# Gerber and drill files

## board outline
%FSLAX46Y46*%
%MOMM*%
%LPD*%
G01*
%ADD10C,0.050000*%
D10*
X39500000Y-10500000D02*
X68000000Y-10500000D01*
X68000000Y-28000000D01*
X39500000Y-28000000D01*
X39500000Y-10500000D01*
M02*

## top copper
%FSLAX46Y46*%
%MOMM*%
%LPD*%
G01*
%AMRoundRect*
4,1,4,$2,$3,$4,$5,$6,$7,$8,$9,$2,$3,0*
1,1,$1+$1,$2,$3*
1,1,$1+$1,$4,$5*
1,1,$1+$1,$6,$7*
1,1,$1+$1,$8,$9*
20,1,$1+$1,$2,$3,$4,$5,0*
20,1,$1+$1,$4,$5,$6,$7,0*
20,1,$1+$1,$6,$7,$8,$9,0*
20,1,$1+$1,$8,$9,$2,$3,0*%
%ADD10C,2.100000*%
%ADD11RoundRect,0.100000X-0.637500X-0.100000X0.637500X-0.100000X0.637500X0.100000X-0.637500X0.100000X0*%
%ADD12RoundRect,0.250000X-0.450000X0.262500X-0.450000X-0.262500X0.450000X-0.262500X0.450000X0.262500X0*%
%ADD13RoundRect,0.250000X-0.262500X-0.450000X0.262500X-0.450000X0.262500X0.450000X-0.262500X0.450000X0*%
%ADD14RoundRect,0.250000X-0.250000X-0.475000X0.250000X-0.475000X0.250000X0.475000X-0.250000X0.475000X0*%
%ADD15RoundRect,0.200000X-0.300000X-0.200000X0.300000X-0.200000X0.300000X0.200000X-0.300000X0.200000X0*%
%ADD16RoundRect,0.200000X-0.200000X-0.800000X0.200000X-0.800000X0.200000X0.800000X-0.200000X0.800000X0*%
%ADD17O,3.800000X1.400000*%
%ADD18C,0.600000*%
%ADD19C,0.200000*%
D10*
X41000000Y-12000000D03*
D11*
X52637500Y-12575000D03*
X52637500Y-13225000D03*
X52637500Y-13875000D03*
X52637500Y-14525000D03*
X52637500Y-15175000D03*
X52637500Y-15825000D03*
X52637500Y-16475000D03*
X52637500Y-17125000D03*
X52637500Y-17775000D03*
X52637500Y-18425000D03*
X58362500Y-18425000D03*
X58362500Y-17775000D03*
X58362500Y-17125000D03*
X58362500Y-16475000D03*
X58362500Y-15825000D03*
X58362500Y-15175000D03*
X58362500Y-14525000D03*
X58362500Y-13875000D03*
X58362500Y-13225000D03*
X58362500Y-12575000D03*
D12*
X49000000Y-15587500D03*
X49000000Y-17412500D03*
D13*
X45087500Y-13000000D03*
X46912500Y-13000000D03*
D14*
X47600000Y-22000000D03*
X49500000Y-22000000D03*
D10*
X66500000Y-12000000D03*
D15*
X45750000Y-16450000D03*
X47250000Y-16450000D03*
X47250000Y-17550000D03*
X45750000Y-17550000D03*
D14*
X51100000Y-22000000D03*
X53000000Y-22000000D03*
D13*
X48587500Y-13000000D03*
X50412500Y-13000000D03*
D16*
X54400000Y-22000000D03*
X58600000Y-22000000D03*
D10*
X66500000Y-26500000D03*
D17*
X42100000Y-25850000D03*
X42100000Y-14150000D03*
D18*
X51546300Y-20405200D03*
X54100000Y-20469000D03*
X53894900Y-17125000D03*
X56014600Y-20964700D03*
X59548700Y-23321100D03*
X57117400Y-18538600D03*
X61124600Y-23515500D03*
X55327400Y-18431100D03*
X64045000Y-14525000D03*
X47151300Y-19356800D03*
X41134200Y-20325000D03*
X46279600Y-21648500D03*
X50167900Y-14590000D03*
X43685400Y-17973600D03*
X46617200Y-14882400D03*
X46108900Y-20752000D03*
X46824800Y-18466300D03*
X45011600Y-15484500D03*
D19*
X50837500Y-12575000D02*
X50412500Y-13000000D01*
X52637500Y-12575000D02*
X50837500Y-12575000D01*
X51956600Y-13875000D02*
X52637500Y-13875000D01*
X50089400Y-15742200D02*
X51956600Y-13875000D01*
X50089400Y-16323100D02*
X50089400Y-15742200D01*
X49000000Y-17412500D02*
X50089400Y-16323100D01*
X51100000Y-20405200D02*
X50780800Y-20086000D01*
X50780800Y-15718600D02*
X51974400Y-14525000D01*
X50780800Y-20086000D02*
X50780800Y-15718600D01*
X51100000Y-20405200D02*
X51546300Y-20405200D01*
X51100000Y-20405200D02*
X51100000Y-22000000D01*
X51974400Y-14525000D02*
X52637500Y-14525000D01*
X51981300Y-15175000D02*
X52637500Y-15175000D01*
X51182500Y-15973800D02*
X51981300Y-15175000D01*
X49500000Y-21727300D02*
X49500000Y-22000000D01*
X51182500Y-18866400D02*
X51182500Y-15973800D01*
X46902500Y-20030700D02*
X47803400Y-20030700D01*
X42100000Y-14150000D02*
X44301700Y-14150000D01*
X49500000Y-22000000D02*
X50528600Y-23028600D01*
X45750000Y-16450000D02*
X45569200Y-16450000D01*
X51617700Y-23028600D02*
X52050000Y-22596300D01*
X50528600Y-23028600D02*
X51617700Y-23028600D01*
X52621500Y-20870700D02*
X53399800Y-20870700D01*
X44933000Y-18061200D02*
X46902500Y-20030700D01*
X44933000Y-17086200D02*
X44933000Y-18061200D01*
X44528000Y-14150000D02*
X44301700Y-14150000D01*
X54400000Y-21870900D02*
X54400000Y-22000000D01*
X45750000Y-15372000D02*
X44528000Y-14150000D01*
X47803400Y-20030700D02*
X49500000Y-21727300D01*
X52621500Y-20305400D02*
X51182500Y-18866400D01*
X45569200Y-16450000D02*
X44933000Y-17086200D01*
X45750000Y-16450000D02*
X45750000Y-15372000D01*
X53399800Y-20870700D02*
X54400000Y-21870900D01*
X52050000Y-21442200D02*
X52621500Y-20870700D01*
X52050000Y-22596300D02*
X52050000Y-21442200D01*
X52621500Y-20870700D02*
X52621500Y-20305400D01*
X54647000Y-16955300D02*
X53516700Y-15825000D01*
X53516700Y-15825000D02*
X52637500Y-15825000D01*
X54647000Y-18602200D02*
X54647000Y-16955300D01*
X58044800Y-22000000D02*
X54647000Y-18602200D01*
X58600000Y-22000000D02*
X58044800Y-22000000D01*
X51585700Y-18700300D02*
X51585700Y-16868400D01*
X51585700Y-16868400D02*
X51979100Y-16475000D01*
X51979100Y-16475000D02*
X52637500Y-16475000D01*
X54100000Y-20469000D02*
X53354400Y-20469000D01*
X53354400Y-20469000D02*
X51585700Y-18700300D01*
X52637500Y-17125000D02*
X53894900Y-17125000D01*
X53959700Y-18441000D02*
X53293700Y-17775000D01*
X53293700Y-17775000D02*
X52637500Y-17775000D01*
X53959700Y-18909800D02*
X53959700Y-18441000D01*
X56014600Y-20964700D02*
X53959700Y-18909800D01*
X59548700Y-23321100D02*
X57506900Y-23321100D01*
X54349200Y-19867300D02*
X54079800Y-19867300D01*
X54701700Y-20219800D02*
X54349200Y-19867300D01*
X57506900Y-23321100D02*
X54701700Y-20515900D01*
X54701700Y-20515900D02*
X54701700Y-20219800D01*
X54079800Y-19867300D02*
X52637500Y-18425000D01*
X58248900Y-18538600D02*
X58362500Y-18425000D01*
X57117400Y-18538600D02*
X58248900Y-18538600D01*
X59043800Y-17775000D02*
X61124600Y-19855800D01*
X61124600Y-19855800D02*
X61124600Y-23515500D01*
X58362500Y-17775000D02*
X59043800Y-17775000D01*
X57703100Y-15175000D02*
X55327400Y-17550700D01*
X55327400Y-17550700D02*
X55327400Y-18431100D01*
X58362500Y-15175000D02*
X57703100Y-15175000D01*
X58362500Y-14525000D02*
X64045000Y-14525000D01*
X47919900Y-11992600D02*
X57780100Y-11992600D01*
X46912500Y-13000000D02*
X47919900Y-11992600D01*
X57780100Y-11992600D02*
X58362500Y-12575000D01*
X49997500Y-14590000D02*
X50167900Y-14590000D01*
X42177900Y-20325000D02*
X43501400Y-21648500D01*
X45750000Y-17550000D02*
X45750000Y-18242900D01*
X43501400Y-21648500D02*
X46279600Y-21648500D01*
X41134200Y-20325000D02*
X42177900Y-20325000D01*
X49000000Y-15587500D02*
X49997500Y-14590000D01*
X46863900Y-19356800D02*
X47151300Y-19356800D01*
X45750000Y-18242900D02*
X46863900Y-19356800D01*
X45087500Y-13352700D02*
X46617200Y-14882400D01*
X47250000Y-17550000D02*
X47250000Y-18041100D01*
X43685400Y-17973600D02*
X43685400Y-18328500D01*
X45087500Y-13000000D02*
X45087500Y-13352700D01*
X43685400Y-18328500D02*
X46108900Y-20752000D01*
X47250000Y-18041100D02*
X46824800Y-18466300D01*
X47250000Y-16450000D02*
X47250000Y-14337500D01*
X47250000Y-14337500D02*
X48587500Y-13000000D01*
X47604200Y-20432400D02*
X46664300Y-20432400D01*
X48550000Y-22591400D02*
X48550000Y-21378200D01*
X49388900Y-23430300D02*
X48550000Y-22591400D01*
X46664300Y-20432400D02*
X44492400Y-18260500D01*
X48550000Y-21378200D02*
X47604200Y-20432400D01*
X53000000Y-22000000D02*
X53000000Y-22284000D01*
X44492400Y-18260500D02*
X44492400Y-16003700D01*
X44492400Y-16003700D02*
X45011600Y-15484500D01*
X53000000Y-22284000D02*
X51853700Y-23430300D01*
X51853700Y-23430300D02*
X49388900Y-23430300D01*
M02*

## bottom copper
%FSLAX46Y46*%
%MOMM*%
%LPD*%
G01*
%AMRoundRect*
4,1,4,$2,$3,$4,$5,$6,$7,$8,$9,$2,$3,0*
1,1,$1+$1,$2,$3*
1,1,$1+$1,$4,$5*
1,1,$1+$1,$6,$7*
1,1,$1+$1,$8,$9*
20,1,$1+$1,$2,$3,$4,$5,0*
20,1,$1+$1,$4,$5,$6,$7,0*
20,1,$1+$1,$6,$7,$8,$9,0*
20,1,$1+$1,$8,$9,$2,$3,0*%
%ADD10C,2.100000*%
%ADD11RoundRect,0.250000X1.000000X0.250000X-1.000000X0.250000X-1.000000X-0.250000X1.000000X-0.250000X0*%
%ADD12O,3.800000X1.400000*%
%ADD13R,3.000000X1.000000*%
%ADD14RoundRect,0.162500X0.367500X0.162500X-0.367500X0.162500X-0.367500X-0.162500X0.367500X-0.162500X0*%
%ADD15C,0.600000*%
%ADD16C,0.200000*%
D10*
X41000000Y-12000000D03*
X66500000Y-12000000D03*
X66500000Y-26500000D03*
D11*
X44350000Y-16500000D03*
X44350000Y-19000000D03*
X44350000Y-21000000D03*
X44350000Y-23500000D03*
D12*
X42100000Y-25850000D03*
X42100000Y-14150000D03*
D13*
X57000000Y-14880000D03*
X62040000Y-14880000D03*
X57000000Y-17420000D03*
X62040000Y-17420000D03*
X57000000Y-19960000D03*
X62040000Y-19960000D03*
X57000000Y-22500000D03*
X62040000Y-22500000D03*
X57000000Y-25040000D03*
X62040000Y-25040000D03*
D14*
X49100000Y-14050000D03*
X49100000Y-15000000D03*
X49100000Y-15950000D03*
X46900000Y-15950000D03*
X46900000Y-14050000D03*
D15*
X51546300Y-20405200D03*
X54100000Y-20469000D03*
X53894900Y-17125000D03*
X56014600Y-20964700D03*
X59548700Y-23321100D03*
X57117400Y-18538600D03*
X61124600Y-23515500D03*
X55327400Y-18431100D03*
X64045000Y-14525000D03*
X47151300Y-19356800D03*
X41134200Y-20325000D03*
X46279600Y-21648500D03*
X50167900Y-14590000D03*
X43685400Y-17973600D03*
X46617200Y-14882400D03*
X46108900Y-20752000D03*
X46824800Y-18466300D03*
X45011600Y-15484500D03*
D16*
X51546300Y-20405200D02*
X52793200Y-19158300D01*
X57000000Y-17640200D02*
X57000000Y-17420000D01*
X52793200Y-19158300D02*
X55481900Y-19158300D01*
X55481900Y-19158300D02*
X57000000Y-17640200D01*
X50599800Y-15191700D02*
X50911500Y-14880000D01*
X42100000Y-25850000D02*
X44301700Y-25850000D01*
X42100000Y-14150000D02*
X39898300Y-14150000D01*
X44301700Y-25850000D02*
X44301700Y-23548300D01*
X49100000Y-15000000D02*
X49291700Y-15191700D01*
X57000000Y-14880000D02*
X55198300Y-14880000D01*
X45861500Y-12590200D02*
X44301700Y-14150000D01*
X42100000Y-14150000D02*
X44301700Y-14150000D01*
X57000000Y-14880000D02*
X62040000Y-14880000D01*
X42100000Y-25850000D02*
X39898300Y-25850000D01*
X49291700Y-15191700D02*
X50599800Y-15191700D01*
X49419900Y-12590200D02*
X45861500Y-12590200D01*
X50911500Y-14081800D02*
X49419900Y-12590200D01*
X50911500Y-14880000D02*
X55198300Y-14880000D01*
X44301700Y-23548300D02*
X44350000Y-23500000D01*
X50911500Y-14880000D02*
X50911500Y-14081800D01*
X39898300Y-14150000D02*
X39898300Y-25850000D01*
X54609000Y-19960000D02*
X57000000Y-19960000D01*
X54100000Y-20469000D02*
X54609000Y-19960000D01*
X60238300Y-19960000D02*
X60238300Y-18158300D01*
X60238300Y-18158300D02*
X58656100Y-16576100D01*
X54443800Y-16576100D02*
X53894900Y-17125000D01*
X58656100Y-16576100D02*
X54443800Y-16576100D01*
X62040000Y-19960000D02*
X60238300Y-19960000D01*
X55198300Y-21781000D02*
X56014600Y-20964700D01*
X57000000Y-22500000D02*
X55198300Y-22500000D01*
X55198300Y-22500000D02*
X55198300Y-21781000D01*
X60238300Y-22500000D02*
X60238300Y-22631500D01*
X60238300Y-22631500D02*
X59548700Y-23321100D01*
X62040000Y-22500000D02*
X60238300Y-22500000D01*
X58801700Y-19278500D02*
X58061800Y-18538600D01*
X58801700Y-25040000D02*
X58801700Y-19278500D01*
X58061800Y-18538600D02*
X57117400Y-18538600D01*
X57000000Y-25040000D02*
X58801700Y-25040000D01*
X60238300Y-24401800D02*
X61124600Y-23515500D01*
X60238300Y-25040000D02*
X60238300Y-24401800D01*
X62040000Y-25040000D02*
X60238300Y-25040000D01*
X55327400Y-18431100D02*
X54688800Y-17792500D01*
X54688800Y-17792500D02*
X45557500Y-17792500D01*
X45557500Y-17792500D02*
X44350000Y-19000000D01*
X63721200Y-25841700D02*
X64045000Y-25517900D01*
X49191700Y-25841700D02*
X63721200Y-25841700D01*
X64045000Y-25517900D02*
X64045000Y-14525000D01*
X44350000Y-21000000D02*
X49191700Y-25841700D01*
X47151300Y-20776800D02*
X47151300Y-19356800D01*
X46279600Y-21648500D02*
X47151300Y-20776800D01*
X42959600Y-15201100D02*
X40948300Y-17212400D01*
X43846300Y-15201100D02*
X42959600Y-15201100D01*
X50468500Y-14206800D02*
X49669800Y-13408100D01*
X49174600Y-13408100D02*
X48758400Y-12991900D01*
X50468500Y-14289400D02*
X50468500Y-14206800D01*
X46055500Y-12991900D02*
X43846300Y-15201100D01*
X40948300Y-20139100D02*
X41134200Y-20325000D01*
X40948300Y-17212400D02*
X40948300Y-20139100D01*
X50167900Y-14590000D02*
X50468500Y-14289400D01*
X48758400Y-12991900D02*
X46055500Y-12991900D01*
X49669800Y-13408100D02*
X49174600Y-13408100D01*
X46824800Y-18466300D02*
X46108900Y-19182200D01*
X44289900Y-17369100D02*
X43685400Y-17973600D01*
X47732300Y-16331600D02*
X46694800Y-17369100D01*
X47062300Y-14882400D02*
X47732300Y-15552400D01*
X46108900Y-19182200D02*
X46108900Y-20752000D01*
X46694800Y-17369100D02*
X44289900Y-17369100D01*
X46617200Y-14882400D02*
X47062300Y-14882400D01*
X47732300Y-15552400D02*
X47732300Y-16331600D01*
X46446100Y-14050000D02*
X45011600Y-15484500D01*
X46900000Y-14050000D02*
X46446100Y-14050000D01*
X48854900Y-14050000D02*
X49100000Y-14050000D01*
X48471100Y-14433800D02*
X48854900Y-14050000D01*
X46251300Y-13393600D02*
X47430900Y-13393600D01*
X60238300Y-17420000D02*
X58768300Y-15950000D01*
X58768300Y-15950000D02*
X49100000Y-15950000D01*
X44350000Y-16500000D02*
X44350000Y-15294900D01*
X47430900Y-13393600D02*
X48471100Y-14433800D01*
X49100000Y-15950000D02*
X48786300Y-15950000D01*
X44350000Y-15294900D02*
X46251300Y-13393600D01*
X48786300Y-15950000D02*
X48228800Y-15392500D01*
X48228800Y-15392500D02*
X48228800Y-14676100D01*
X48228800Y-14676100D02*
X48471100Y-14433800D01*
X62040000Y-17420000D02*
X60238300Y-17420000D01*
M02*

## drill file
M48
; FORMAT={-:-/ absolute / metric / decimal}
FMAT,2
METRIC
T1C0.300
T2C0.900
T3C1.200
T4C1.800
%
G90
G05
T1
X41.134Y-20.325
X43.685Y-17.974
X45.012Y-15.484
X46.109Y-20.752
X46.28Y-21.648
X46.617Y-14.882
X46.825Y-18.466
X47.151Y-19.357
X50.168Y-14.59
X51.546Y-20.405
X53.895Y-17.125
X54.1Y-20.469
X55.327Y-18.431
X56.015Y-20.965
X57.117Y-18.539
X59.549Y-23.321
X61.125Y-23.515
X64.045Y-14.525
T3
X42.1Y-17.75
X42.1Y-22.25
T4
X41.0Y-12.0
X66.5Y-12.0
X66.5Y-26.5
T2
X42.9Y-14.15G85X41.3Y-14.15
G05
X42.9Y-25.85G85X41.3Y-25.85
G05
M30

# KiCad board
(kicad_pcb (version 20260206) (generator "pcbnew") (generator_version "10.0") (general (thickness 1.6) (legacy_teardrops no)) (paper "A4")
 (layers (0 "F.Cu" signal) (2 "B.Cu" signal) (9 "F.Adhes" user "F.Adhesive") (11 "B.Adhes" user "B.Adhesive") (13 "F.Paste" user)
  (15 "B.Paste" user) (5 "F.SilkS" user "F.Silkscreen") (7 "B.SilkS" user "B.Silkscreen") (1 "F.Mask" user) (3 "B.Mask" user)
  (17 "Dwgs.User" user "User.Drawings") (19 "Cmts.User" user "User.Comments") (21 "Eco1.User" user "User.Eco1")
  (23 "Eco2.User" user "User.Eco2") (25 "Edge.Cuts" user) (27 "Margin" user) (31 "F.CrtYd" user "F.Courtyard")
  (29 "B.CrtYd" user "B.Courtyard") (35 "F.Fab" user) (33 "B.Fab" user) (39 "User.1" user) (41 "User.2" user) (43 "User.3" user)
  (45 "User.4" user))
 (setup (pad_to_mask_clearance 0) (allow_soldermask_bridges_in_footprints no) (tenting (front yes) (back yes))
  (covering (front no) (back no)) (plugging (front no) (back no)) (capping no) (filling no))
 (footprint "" (layer "F.Cu") (at 41 12)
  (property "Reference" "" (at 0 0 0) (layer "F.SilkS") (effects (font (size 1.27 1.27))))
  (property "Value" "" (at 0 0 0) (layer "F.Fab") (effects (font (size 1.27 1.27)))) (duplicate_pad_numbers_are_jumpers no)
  (pad "" np_thru_hole circle (at 0 0) (size 2.1 2.1) (drill 1.8) (layers "*.Cu" "*.Mask")))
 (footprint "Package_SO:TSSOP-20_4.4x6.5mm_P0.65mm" (layer "F.Cu") (at 55.5 15.5)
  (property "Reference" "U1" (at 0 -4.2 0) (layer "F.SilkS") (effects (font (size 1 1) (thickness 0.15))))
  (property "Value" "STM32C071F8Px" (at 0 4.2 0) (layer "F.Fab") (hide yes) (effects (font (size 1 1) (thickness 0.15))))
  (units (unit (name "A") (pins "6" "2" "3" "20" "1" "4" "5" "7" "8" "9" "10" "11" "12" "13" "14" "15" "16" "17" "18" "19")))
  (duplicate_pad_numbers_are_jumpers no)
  (pad "1" smd roundrect (at -2.8625 -2.925) (size 1.475 0.4) (layers "F.Cu" "F.Mask" "F.Paste") (roundrect_rratio 0.25)
   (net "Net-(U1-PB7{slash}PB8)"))
  (pad "2" smd roundrect (at -2.8625 -2.275) (size 1.475 0.4) (layers "F.Cu" "F.Mask" "F.Paste") (roundrect_rratio 0.25)
   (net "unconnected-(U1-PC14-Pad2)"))
  (pad "3" smd roundrect (at -2.8625 -1.625) (size 1.475 0.4) (layers "F.Cu" "F.Mask" "F.Paste") (roundrect_rratio 0.25)
   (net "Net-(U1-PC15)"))
  (pad "4" smd roundrect (at -2.8625 -0.975) (size 1.475 0.4) (layers "F.Cu" "F.Mask" "F.Paste") (roundrect_rratio 0.25)
   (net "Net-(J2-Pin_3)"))
  (pad "5" smd roundrect (at -2.8625 -0.325) (size 1.475 0.4) (layers "F.Cu" "F.Mask" "F.Paste") (roundrect_rratio 0.25)
   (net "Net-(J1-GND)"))
  (pad "6" smd roundrect (at -2.8625 0.325) (size 1.475 0.4) (layers "F.Cu" "F.Mask" "F.Paste") (roundrect_rratio 0.25) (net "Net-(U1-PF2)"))
  (pad "7" smd roundrect (at -2.8625 0.975) (size 1.475 0.4) (layers "F.Cu" "F.Mask" "F.Paste") (roundrect_rratio 0.25)
   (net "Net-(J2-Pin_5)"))
  (pad "8" smd roundrect (at -2.8625 1.625) (size 1.475 0.4) (layers "F.Cu" "F.Mask" "F.Paste") (roundrect_rratio 0.25)
   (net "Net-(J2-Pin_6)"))
  (pad "9" smd roundrect (at -2.8625 2.275) (size 1.475 0.4) (layers "F.Cu" "F.Mask" "F.Paste") (roundrect_rratio 0.25)
   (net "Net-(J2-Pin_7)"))
  (pad "10" smd roundrect (at -2.8625 2.925) (size 1.475 0.4) (layers "F.Cu" "F.Mask" "F.Paste") (roundrect_rratio 0.25)
   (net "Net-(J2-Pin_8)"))
  (pad "11" smd roundrect (at 2.8625 2.925) (size 1.475 0.4) (layers "F.Cu" "F.Mask" "F.Paste") (roundrect_rratio 0.25)
   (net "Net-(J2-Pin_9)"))
  (pad "12" smd roundrect (at 2.8625 2.275) (size 1.475 0.4) (layers "F.Cu" "F.Mask" "F.Paste") (roundrect_rratio 0.25)
   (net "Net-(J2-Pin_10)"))
  (pad "13" smd roundrect (at 2.8625 1.625) (size 1.475 0.4) (layers "F.Cu" "F.Mask" "F.Paste") (roundrect_rratio 0.25)
   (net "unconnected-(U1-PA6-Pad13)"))
  (pad "14" smd roundrect (at 2.8625 0.975) (size 1.475 0.4) (layers "F.Cu" "F.Mask" "F.Paste") (roundrect_rratio 0.25)
   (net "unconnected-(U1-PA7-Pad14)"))
  (pad "15" smd roundrect (at 2.8625 0.325) (size 1.475 0.4) (layers "F.Cu" "F.Mask" "F.Paste") (roundrect_rratio 0.25)
   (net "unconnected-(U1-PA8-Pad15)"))
  (pad "16" smd roundrect (at 2.8625 -0.325) (size 1.475 0.4) (layers "F.Cu" "F.Mask" "F.Paste") (roundrect_rratio 0.25) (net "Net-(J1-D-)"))
  (pad "17" smd roundrect (at 2.8625 -0.975) (size 1.475 0.4) (layers "F.Cu" "F.Mask" "F.Paste") (roundrect_rratio 0.25) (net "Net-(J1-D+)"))
  (pad "18" smd roundrect (at 2.8625 -1.625) (size 1.475 0.4) (layers "F.Cu" "F.Mask" "F.Paste") (roundrect_rratio 0.25)
   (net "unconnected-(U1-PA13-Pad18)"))
  (pad "19" smd roundrect (at 2.8625 -2.275) (size 1.475 0.4) (layers "F.Cu" "F.Mask" "F.Paste") (roundrect_rratio 0.25)
   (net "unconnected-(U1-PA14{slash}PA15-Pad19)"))
  (pad "20" smd roundrect (at 2.8625 -2.925) (size 1.475 0.4) (layers "F.Cu" "F.Mask" "F.Paste") (roundrect_rratio 0.25)
   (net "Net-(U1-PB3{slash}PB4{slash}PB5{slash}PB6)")))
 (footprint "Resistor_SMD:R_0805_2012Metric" (layer "F.Cu") (at 49 16.5 -90)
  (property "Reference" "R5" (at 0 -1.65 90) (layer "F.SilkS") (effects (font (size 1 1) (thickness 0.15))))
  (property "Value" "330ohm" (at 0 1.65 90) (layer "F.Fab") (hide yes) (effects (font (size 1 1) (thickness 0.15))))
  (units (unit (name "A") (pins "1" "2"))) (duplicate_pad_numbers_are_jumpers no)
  (pad "1" smd roundrect (at -0.9125 0 270) (size 1.025 1.4) (layers "F.Cu" "F.Mask" "F.Paste") (roundrect_rratio 0.243902)
   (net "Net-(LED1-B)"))
  (pad "2" smd roundrect (at 0.9125 0 270) (size 1.025 1.4) (layers "F.Cu" "F.Mask" "F.Paste") (roundrect_rratio 0.243902)
   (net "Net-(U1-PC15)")))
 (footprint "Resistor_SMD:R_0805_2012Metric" (layer "F.Cu") (at 46 13)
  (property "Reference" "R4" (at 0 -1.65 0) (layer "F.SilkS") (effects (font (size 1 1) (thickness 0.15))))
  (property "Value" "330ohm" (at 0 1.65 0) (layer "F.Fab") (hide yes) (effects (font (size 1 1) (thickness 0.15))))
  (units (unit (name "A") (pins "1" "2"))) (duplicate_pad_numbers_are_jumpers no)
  (pad "1" smd roundrect (at -0.9125 0) (size 1.025 1.4) (layers "F.Cu" "F.Mask" "F.Paste") (roundrect_rratio 0.243902) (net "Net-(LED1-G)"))
  (pad "2" smd roundrect (at 0.9125 0) (size 1.025 1.4) (layers "F.Cu" "F.Mask" "F.Paste") (roundrect_rratio 0.243902)
   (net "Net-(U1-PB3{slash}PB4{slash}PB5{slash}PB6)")))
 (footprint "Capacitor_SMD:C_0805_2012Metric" (layer "F.Cu") (at 48.55 22)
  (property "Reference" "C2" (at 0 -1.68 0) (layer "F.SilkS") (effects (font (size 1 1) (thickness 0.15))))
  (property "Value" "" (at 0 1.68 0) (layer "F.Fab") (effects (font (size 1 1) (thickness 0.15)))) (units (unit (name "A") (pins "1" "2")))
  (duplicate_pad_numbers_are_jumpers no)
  (pad "1" smd roundrect (at -0.95 0) (size 1 1.45) (layers "F.Cu" "F.Mask" "F.Paste") (roundrect_rratio 0.25) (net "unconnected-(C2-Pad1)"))
  (pad "2" smd roundrect (at 0.95 0) (size 1 1.45) (layers "F.Cu" "F.Mask" "F.Paste") (roundrect_rratio 0.25) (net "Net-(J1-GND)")))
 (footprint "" (layer "F.Cu") (at 66.5 12)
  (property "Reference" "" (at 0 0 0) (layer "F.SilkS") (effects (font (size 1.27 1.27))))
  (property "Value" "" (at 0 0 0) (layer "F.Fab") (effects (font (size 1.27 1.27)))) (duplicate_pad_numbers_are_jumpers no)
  (pad "" np_thru_hole circle (at 0 0) (size 2.1 2.1) (drill 1.8) (layers "*.Cu" "*.Mask")))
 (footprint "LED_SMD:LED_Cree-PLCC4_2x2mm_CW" (layer "F.Cu") (at 46.5 17)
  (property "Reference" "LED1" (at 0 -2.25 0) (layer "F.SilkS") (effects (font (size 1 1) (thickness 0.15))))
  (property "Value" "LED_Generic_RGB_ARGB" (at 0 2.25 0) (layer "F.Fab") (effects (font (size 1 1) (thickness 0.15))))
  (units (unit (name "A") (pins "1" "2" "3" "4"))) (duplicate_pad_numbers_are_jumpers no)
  (pad "1" smd roundrect (at -0.75 -0.55) (size 1 0.8) (layers "F.Cu" "F.Mask" "F.Paste") (roundrect_rratio 0.25) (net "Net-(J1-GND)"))
  (pad "2" smd roundrect (at 0.75 -0.55) (size 1 0.8) (layers "F.Cu" "F.Mask" "F.Paste") (roundrect_rratio 0.25) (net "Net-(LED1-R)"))
  (pad "3" smd roundrect (at 0.75 0.55) (size 1 0.8) (layers "F.Cu" "F.Mask" "F.Paste") (roundrect_rratio 0.25) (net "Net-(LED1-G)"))
  (pad "4" smd roundrect (at -0.75 0.55) (size 1 0.8) (layers "F.Cu" "F.Mask" "F.Paste") (roundrect_rratio 0.25) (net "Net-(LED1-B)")))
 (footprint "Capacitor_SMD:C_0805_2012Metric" (layer "F.Cu") (at 52.05 22)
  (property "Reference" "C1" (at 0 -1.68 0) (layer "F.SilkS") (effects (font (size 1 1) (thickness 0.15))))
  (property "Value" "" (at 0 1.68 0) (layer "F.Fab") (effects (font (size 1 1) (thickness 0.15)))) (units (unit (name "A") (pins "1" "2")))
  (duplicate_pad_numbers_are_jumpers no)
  (pad "1" smd roundrect (at -0.95 0) (size 1 1.45) (layers "F.Cu" "F.Mask" "F.Paste") (roundrect_rratio 0.25) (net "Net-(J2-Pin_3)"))
  (pad "2" smd roundrect (at 0.95 0) (size 1 1.45) (layers "F.Cu" "F.Mask" "F.Paste") (roundrect_rratio 0.25) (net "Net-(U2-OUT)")))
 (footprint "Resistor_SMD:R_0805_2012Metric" (layer "F.Cu") (at 49.5 13)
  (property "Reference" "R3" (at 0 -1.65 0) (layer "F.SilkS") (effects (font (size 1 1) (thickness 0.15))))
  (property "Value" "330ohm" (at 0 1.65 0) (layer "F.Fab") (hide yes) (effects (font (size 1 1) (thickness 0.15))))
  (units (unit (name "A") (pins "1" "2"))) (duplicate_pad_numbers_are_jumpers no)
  (pad "1" smd roundrect (at -0.9125 0) (size 1.025 1.4) (layers "F.Cu" "F.Mask" "F.Paste") (roundrect_rratio 0.243902) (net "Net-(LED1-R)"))
  (pad "2" smd roundrect (at 0.9125 0) (size 1.025 1.4) (layers "F.Cu" "F.Mask" "F.Paste") (roundrect_rratio 0.243902)
   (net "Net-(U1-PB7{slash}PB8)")))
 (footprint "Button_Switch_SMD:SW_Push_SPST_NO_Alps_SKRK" (layer "F.Cu") (at 56.5 22)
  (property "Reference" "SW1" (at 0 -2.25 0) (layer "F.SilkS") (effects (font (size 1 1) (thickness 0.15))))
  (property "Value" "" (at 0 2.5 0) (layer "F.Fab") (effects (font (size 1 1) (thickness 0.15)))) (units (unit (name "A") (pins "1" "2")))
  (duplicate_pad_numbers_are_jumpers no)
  (pad "1" smd roundrect (at -2.1 0) (size 0.8 2) (layers "F.Cu" "F.Mask" "F.Paste") (roundrect_rratio 0.25) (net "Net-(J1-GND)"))
  (pad "2" smd roundrect (at 2.1 0) (size 0.8 2) (layers "F.Cu" "F.Mask" "F.Paste") (roundrect_rratio 0.25) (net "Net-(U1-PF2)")))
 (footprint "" (layer "F.Cu") (at 66.5 26.5)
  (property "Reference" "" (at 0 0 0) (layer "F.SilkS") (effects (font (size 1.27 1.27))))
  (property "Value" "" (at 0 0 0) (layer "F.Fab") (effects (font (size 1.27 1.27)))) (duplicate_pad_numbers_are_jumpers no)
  (pad "" np_thru_hole circle (at 0 0) (size 2.1 2.1) (drill 1.8) (layers "*.Cu" "*.Mask")))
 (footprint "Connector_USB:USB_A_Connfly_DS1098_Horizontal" (layer "B.Cu") (at 33.8 20 180)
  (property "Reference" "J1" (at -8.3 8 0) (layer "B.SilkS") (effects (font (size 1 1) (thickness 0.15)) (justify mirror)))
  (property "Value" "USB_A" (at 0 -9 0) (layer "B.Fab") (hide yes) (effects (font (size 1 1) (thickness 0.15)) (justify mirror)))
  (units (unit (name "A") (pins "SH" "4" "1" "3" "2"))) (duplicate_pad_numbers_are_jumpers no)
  (pad "" np_thru_hole circle (at -8.3 -2.25 180) (size 1.2 1.2) (drill 1.2) (layers "*.Mask"))
  (pad "" np_thru_hole circle (at -8.3 2.25 180) (size 1.2 1.2) (drill 1.2) (layers "*.Mask"))
  (pad "1" smd roundrect (at -10.55 3.5 180) (size 2.5 1) (layers "B.Cu" "B.Mask" "B.Paste") (roundrect_rratio 0.25) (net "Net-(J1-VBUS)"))
  (pad "2" smd roundrect (at -10.55 1 180) (size 2.5 1) (layers "B.Cu" "B.Mask" "B.Paste") (roundrect_rratio 0.25) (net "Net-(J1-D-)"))
  (pad "3" smd roundrect (at -10.55 -1 180) (size 2.5 1) (layers "B.Cu" "B.Mask" "B.Paste") (roundrect_rratio 0.25) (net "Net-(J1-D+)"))
  (pad "4" smd roundrect (at -10.55 -3.5 180) (size 2.5 1) (layers "B.Cu" "B.Mask" "B.Paste") (roundrect_rratio 0.25) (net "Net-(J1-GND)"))
  (pad "SH" thru_hole oval (at -8.3 -5.85 180) (size 3.8 1.4) (drill oval 2.5 0.9) (layers "*.Cu" "*.Mask") (remove_unused_layers no)
   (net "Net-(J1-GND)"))
  (pad "SH" thru_hole oval (at -8.3 5.85 180) (size 3.8 1.4) (drill oval 2.5 0.9) (layers "*.Cu" "*.Mask") (remove_unused_layers no)
   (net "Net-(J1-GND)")))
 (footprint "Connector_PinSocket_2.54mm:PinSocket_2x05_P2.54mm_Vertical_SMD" (layer "B.Cu") (at 59.52 19.96 180)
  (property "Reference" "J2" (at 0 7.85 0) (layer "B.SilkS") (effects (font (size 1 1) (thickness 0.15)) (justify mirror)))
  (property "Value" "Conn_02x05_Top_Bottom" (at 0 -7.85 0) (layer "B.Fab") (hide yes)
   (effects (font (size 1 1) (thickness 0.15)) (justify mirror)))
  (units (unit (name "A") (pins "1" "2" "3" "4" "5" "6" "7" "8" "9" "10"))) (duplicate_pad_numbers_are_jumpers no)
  (pad "1" smd rect (at 2.52 5.08 180) (size 3 1) (layers "B.Cu" "B.Mask" "B.Paste") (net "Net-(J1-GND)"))
  (pad "2" smd rect (at -2.52 5.08 180) (size 3 1) (layers "B.Cu" "B.Mask" "B.Paste") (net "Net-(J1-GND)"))
  (pad "3" smd rect (at 2.52 2.54 180) (size 3 1) (layers "B.Cu" "B.Mask" "B.Paste") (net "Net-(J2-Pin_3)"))
  (pad "4" smd rect (at -2.52 2.54 180) (size 3 1) (layers "B.Cu" "B.Mask" "B.Paste") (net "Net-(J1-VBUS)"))
  (pad "5" smd rect (at 2.52 0 180) (size 3 1) (layers "B.Cu" "B.Mask" "B.Paste") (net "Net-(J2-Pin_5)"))
  (pad "6" smd rect (at -2.52 0 180) (size 3 1) (layers "B.Cu" "B.Mask" "B.Paste") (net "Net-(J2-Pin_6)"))
  (pad "7" smd rect (at 2.52 -2.54 180) (size 3 1) (layers "B.Cu" "B.Mask" "B.Paste") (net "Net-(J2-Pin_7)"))
  (pad "8" smd rect (at -2.52 -2.54 180) (size 3 1) (layers "B.Cu" "B.Mask" "B.Paste") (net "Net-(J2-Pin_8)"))
  (pad "9" smd rect (at 2.52 -5.08 180) (size 3 1) (layers "B.Cu" "B.Mask" "B.Paste") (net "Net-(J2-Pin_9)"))
  (pad "10" smd rect (at -2.52 -5.08 180) (size 3 1) (layers "B.Cu" "B.Mask" "B.Paste") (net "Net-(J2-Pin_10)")))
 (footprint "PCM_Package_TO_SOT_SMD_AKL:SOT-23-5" (layer "B.Cu") (at 48 15 180)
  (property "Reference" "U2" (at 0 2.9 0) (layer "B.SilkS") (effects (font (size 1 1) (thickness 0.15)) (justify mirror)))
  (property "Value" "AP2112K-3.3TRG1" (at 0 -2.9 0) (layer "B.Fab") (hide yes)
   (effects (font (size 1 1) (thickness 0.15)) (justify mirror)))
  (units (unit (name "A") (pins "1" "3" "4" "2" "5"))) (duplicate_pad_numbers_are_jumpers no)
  (pad "1" smd roundrect (at -1.1 0.95 180) (size 1.06 0.65) (layers "B.Cu" "B.Mask" "B.Paste") (roundrect_rratio 0.25)
   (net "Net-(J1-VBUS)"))
  (pad "2" smd roundrect (at -1.1 0 180) (size 1.06 0.65) (layers "B.Cu" "B.Mask" "B.Paste") (roundrect_rratio 0.25) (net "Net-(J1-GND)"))
  (pad "3" smd roundrect (at -1.1 -0.95 180) (size 1.06 0.65) (layers "B.Cu" "B.Mask" "B.Paste") (roundrect_rratio 0.25)
   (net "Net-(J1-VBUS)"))
  (pad "4" smd roundrect (at 1.1 -0.95 180) (size 1.06 0.65) (layers "B.Cu" "B.Mask" "B.Paste") (roundrect_rratio 0.25)
   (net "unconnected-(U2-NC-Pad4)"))
  (pad "5" smd roundrect (at 1.1 0.95 180) (size 1.06 0.65) (layers "B.Cu" "B.Mask" "B.Paste") (roundrect_rratio 0.25) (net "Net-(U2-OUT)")))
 (gr_rect (start 39.5 10.5) (end 68 28) (stroke (width 0.05) (type default)) (fill no) (layer "Edge.Cuts"))
 (segment (start 50.8375 12.575) (end 50.4125 13) (width 0.2) (layer "F.Cu") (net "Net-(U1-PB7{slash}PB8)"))
 (segment (start 52.6375 12.575) (end 50.8375 12.575) (width 0.2) (layer "F.Cu") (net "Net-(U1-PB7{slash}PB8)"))
 (segment (start 51.9566 13.875) (end 52.6375 13.875) (width 0.2) (layer "F.Cu") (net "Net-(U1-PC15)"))
 (segment (start 50.0894 15.7422) (end 51.9566 13.875) (width 0.2) (layer "F.Cu") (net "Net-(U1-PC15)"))
 (segment (start 50.0894 16.3231) (end 50.0894 15.7422) (width 0.2) (layer "F.Cu") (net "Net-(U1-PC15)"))
 (segment (start 49 17.4125) (end 50.0894 16.3231) (width 0.2) (layer "F.Cu") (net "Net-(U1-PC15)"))
 (segment (start 51.1 20.4052) (end 50.7808 20.086) (width 0.2) (layer "F.Cu") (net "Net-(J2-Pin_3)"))
 (segment (start 50.7808 15.7186) (end 51.9744 14.525) (width 0.2) (layer "F.Cu") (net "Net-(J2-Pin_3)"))
 (segment (start 50.7808 20.086) (end 50.7808 15.7186) (width 0.2) (layer "F.Cu") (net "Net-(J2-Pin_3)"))
 (segment (start 51.1 20.4052) (end 51.5463 20.4052) (width 0.2) (layer "F.Cu") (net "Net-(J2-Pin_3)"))
 (segment (start 51.1 20.4052) (end 51.1 22) (width 0.2) (layer "F.Cu") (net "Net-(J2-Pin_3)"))
 (segment (start 51.9744 14.525) (end 52.6375 14.525) (width 0.2) (layer "F.Cu") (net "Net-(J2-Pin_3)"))
 (via (at 51.5463 20.4052) (size 0.6) (drill 0.3) (layers "F.Cu" "B.Cu") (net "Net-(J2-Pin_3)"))
 (segment (start 51.5463 20.4052) (end 52.7932 19.1583) (width 0.2) (layer "B.Cu") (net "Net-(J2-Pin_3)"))
 (segment (start 57 17.6402) (end 57 17.42) (width 0.2) (layer "B.Cu") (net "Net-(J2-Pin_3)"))
 (segment (start 52.7932 19.1583) (end 55.4819 19.1583) (width 0.2) (layer "B.Cu") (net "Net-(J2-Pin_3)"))
 (segment (start 55.4819 19.1583) (end 57 17.6402) (width 0.2) (layer "B.Cu") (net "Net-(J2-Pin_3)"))
 (segment (start 51.9813 15.175) (end 52.6375 15.175) (width 0.2) (layer "F.Cu") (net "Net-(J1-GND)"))
 (segment (start 51.1825 15.9738) (end 51.9813 15.175) (width 0.2) (layer "F.Cu") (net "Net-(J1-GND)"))
 (segment (start 49.5 21.7273) (end 49.5 22) (width 0.2) (layer "F.Cu") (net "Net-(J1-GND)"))
 (segment (start 51.1825 18.8664) (end 51.1825 15.9738) (width 0.2) (layer "F.Cu") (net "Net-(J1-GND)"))
 (segment (start 46.9025 20.0307) (end 47.8034 20.0307) (width 0.2) (layer "F.Cu") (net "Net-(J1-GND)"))
 (segment (start 42.1 14.15) (end 44.3017 14.15) (width 0.2) (layer "F.Cu") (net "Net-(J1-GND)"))
 (segment (start 49.5 22) (end 50.5286 23.0286) (width 0.2) (layer "F.Cu") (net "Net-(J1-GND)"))
 (segment (start 45.75 16.45) (end 45.5692 16.45) (width 0.2) (layer "F.Cu") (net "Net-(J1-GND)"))
 (segment (start 51.6177 23.0286) (end 52.05 22.5963) (width 0.2) (layer "F.Cu") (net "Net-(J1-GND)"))
 (segment (start 50.5286 23.0286) (end 51.6177 23.0286) (width 0.2) (layer "F.Cu") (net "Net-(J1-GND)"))
 (segment (start 52.6215 20.8707) (end 53.3998 20.8707) (width 0.2) (layer "F.Cu") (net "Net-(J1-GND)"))
 (segment (start 44.933 18.0612) (end 46.9025 20.0307) (width 0.2) (layer "F.Cu") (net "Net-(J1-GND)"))
 (segment (start 44.933 17.0862) (end 44.933 18.0612) (width 0.2) (layer "F.Cu") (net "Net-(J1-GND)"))
 (segment (start 44.528 14.15) (end 44.3017 14.15) (width 0.2) (layer "F.Cu") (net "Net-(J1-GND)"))
 (segment (start 54.4 21.8709) (end 54.4 22) (width 0.2) (layer "F.Cu") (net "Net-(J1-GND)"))
 (segment (start 45.75 15.372) (end 44.528 14.15) (width 0.2) (layer "F.Cu") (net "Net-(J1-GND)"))
 (segment (start 47.8034 20.0307) (end 49.5 21.7273) (width 0.2) (layer "F.Cu") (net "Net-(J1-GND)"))
 (segment (start 52.6215 20.3054) (end 51.1825 18.8664) (width 0.2) (layer "F.Cu") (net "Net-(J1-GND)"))
 (segment (start 45.5692 16.45) (end 44.933 17.0862) (width 0.2) (layer "F.Cu") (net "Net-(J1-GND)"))
 (segment (start 45.75 16.45) (end 45.75 15.372) (width 0.2) (layer "F.Cu") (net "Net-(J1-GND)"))
 (segment (start 53.3998 20.8707) (end 54.4 21.8709) (width 0.2) (layer "F.Cu") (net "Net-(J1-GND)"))
 (segment (start 52.05 21.4422) (end 52.6215 20.8707) (width 0.2) (layer "F.Cu") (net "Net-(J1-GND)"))
 (segment (start 52.05 22.5963) (end 52.05 21.4422) (width 0.2) (layer "F.Cu") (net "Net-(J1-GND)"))
 (segment (start 52.6215 20.8707) (end 52.6215 20.3054) (width 0.2) (layer "F.Cu") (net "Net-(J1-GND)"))
 (segment (start 50.5998 15.1917) (end 50.9115 14.88) (width 0.2) (layer "B.Cu") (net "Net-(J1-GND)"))
 (segment (start 42.1 25.85) (end 44.3017 25.85) (width 0.2) (layer "B.Cu") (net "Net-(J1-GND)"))
 (segment (start 42.1 14.15) (end 39.8983 14.15) (width 0.2) (layer "B.Cu") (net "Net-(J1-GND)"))
 (segment (start 44.3017 25.85) (end 44.3017 23.5483) (width 0.2) (layer "B.Cu") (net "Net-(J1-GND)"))
 (segment (start 49.1 15) (end 49.2917 15.1917) (width 0.2) (layer "B.Cu") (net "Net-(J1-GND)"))
 (segment (start 57 14.88) (end 55.1983 14.88) (width 0.2) (layer "B.Cu") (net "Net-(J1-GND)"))
 (segment (start 45.8615 12.5902) (end 44.3017 14.15) (width 0.2) (layer "B.Cu") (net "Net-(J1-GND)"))
 (segment (start 42.1 14.15) (end 44.3017 14.15) (width 0.2) (layer "B.Cu") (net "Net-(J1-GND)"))
 (segment (start 57 14.88) (end 62.04 14.88) (width 0.2) (layer "B.Cu") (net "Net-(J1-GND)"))
 (segment (start 42.1 25.85) (end 39.8983 25.85) (width 0.2) (layer "B.Cu") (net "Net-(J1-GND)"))
 (segment (start 49.2917 15.1917) (end 50.5998 15.1917) (width 0.2) (layer "B.Cu") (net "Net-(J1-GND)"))
 (segment (start 49.4199 12.5902) (end 45.8615 12.5902) (width 0.2) (layer "B.Cu") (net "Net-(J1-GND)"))
 (segment (start 50.9115 14.0818) (end 49.4199 12.5902) (width 0.2) (layer "B.Cu") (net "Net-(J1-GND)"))
 (segment (start 50.9115 14.88) (end 55.1983 14.88) (width 0.2) (layer "B.Cu") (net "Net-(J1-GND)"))
 (segment (start 44.3017 23.5483) (end 44.35 23.5) (width 0.2) (layer "B.Cu") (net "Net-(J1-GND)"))
 (segment (start 50.9115 14.88) (end 50.9115 14.0818) (width 0.2) (layer "B.Cu") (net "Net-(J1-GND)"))
 (segment (start 39.8983 14.15) (end 39.8983 25.85) (width 0.2) (layer "B.Cu") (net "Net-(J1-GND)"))
 (segment (start 54.647 16.9553) (end 53.5167 15.825) (width 0.2) (layer "F.Cu") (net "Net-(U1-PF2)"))
 (segment (start 53.5167 15.825) (end 52.6375 15.825) (width 0.2) (layer "F.Cu") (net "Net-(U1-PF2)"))
 (segment (start 54.647 18.6022) (end 54.647 16.9553) (width 0.2) (layer "F.Cu") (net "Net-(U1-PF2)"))
 (segment (start 58.0448 22) (end 54.647 18.6022) (width 0.2) (layer "F.Cu") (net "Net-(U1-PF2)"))
 (segment (start 58.6 22) (end 58.0448 22) (width 0.2) (layer "F.Cu") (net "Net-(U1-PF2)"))
 (segment (start 51.5857 18.7003) (end 51.5857 16.8684) (width 0.2) (layer "F.Cu") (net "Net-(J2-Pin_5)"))
 (segment (start 51.5857 16.8684) (end 51.9791 16.475) (width 0.2) (layer "F.Cu") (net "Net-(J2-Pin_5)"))
 (segment (start 51.9791 16.475) (end 52.6375 16.475) (width 0.2) (layer "F.Cu") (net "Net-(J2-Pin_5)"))
 (segment (start 54.1 20.469) (end 53.3544 20.469) (width 0.2) (layer "F.Cu") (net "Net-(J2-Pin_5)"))
 (segment (start 53.3544 20.469) (end 51.5857 18.7003) (width 0.2) (layer "F.Cu") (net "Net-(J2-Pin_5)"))
 (via (at 54.1 20.469) (size 0.6) (drill 0.3) (layers "F.Cu" "B.Cu") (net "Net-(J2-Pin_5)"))
 (segment (start 54.609 19.96) (end 57 19.96) (width 0.2) (layer "B.Cu") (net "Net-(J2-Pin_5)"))
 (segment (start 54.1 20.469) (end 54.609 19.96) (width 0.2) (layer "B.Cu") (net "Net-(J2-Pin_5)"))
 (segment (start 52.6375 17.125) (end 53.8949 17.125) (width 0.2) (layer "F.Cu") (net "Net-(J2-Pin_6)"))
 (via (at 53.8949 17.125) (size 0.6) (drill 0.3) (layers "F.Cu" "B.Cu") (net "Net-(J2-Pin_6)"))
 (segment (start 60.2383 19.96) (end 60.2383 18.1583) (width 0.2) (layer "B.Cu") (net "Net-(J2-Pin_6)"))
 (segment (start 60.2383 18.1583) (end 58.6561 16.5761) (width 0.2) (layer "B.Cu") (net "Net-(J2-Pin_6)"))
 (segment (start 54.4438 16.5761) (end 53.8949 17.125) (width 0.2) (layer "B.Cu") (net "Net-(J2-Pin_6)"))
 (segment (start 58.6561 16.5761) (end 54.4438 16.5761) (width 0.2) (layer "B.Cu") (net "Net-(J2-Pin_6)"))
 (segment (start 62.04 19.96) (end 60.2383 19.96) (width 0.2) (layer "B.Cu") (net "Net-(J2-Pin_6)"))
 (segment (start 53.9597 18.441) (end 53.2937 17.775) (width 0.2) (layer "F.Cu") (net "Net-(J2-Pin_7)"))
 (segment (start 53.2937 17.775) (end 52.6375 17.775) (width 0.2) (layer "F.Cu") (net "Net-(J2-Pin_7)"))
 (segment (start 53.9597 18.9098) (end 53.9597 18.441) (width 0.2) (layer "F.Cu") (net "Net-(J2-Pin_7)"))
 (segment (start 56.0146 20.9647) (end 53.9597 18.9098) (width 0.2) (layer "F.Cu") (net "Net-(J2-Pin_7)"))
 (via (at 56.0146 20.9647) (size 0.6) (drill 0.3) (layers "F.Cu" "B.Cu") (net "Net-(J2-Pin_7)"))
 (segment (start 55.1983 21.781) (end 56.0146 20.9647) (width 0.2) (layer "B.Cu") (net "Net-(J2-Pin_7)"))
 (segment (start 57 22.5) (end 55.1983 22.5) (width 0.2) (layer "B.Cu") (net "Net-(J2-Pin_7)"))
 (segment (start 55.1983 22.5) (end 55.1983 21.781) (width 0.2) (layer "B.Cu") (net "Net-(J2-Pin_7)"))
 (segment (start 59.5487 23.3211) (end 57.5069 23.3211) (width 0.2) (layer "F.Cu") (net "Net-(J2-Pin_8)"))
 (segment (start 54.3492 19.8673) (end 54.0798 19.8673) (width 0.2) (layer "F.Cu") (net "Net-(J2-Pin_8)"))
 (segment (start 54.7017 20.2198) (end 54.3492 19.8673) (width 0.2) (layer "F.Cu") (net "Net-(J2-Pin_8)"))
 (segment (start 57.5069 23.3211) (end 54.7017 20.5159) (width 0.2) (layer "F.Cu") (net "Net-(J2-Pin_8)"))
 (segment (start 54.7017 20.5159) (end 54.7017 20.2198) (width 0.2) (layer "F.Cu") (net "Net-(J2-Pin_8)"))
 (segment (start 54.0798 19.8673) (end 52.6375 18.425) (width 0.2) (layer "F.Cu") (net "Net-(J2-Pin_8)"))
 (via (at 59.5487 23.3211) (size 0.6) (drill 0.3) (layers "F.Cu" "B.Cu") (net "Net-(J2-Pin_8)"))
 (segment (start 60.2383 22.5) (end 60.2383 22.6315) (width 0.2) (layer "B.Cu") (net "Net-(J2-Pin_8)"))
 (segment (start 60.2383 22.6315) (end 59.5487 23.3211) (width 0.2) (layer "B.Cu") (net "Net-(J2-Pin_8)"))
 (segment (start 62.04 22.5) (end 60.2383 22.5) (width 0.2) (layer "B.Cu") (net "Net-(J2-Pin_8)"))
 (segment (start 58.2489 18.5386) (end 58.3625 18.425) (width 0.2) (layer "F.Cu") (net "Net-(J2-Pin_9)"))
 (segment (start 57.1174 18.5386) (end 58.2489 18.5386) (width 0.2) (layer "F.Cu") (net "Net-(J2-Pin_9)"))
 (via (at 57.1174 18.5386) (size 0.6) (drill 0.3) (layers "F.Cu" "B.Cu") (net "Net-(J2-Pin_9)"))
 (segment (start 58.8017 19.2785) (end 58.0618 18.5386) (width 0.2) (layer "B.Cu") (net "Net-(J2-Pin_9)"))
 (segment (start 58.8017 25.04) (end 58.8017 19.2785) (width 0.2) (layer "B.Cu") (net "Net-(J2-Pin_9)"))
 (segment (start 58.0618 18.5386) (end 57.1174 18.5386) (width 0.2) (layer "B.Cu") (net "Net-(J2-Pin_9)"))
 (segment (start 57 25.04) (end 58.8017 25.04) (width 0.2) (layer "B.Cu") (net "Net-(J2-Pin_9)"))
 (segment (start 59.0438 17.775) (end 61.1246 19.8558) (width 0.2) (layer "F.Cu") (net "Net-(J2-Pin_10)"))
 (segment (start 61.1246 19.8558) (end 61.1246 23.5155) (width 0.2) (layer "F.Cu") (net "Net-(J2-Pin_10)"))
 (segment (start 58.3625 17.775) (end 59.0438 17.775) (width 0.2) (layer "F.Cu") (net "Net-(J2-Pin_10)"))
 (via (at 61.1246 23.5155) (size 0.6) (drill 0.3) (layers "F.Cu" "B.Cu") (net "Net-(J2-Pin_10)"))
 (segment (start 60.2383 24.4018) (end 61.1246 23.5155) (width 0.2) (layer "B.Cu") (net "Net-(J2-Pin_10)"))
 (segment (start 60.2383 25.04) (end 60.2383 24.4018) (width 0.2) (layer "B.Cu") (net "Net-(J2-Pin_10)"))
 (segment (start 62.04 25.04) (end 60.2383 25.04) (width 0.2) (layer "B.Cu") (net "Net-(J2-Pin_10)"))
 (segment (start 57.7031 15.175) (end 55.3274 17.5507) (width 0.2) (layer "F.Cu") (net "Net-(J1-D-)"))
 (segment (start 55.3274 17.5507) (end 55.3274 18.4311) (width 0.2) (layer "F.Cu") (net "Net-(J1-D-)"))
 (segment (start 58.3625 15.175) (end 57.7031 15.175) (width 0.2) (layer "F.Cu") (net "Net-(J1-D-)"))
 (via (at 55.3274 18.4311) (size 0.6) (drill 0.3) (layers "F.Cu" "B.Cu") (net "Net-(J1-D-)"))
 (segment (start 55.3274 18.4311) (end 54.6888 17.7925) (width 0.2) (layer "B.Cu") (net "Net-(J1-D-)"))
 (segment (start 54.6888 17.7925) (end 45.5575 17.7925) (width 0.2) (layer "B.Cu") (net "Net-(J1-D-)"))
 (segment (start 45.5575 17.7925) (end 44.35 19) (width 0.2) (layer "B.Cu") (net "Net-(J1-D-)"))
 (segment (start 58.3625 14.525) (end 64.045 14.525) (width 0.2) (layer "F.Cu") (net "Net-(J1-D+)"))
 (via (at 64.045 14.525) (size 0.6) (drill 0.3) (layers "F.Cu" "B.Cu") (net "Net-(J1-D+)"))
 (segment (start 63.7212 25.8417) (end 64.045 25.5179) (width 0.2) (layer "B.Cu") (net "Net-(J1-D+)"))
 (segment (start 49.1917 25.8417) (end 63.7212 25.8417) (width 0.2) (layer "B.Cu") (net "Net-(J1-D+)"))
 (segment (start 64.045 25.5179) (end 64.045 14.525) (width 0.2) (layer "B.Cu") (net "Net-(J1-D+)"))
 (segment (start 44.35 21) (end 49.1917 25.8417) (width 0.2) (layer "B.Cu") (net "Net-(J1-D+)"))
 (segment (start 47.9199 11.9926) (end 57.7801 11.9926) (width 0.2) (layer "F.Cu") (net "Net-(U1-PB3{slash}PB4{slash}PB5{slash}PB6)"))
 (segment (start 46.9125 13) (end 47.9199 11.9926) (width 0.2) (layer "F.Cu") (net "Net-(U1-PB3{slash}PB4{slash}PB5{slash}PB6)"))
 (segment (start 57.7801 11.9926) (end 58.3625 12.575) (width 0.2) (layer "F.Cu") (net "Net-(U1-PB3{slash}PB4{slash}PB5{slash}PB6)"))
 (segment (start 49.9975 14.59) (end 50.1679 14.59) (width 0.2) (layer "F.Cu") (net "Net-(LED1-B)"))
 (segment (start 42.1779 20.325) (end 43.5014 21.6485) (width 0.2) (layer "F.Cu") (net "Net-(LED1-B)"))
 (segment (start 45.75 17.55) (end 45.75 18.2429) (width 0.2) (layer "F.Cu") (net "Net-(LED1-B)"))
 (segment (start 43.5014 21.6485) (end 46.2796 21.6485) (width 0.2) (layer "F.Cu") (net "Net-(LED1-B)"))
 (segment (start 41.1342 20.325) (end 42.1779 20.325) (width 0.2) (layer "F.Cu") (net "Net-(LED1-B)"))
 (segment (start 49 15.5875) (end 49.9975 14.59) (width 0.2) (layer "F.Cu") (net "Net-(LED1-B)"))
 (segment (start 46.8639 19.3568) (end 47.1513 19.3568) (width 0.2) (layer "F.Cu") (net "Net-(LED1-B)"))
 (segment (start 45.75 18.2429) (end 46.8639 19.3568) (width 0.2) (layer "F.Cu") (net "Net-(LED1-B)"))
 (via (at 47.1513 19.3568) (size 0.6) (drill 0.3) (layers "F.Cu" "B.Cu") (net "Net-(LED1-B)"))
 (via (at 41.1342 20.325) (size 0.6) (drill 0.3) (layers "F.Cu" "B.Cu") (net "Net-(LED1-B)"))
 (via (at 46.2796 21.6485) (size 0.6) (drill 0.3) (layers "F.Cu" "B.Cu") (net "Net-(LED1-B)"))
 (via (at 50.1679 14.59) (size 0.6) (drill 0.3) (layers "F.Cu" "B.Cu") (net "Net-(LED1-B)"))
 (segment (start 47.1513 20.7768) (end 47.1513 19.3568) (width 0.2) (layer "B.Cu") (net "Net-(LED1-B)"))
 (segment (start 46.2796 21.6485) (end 47.1513 20.7768) (width 0.2) (layer "B.Cu") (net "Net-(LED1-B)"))
 (segment (start 42.9596 15.2011) (end 40.9483 17.2124) (width 0.2) (layer "B.Cu") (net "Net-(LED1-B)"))
 (segment (start 43.8463 15.2011) (end 42.9596 15.2011) (width 0.2) (layer "B.Cu") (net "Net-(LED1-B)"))
 (segment (start 50.4685 14.2068) (end 49.6698 13.4081) (width 0.2) (layer "B.Cu") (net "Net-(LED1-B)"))
 (segment (start 49.1746 13.4081) (end 48.7584 12.9919) (width 0.2) (layer "B.Cu") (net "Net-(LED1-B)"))
 (segment (start 50.4685 14.2894) (end 50.4685 14.2068) (width 0.2) (layer "B.Cu") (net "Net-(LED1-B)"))
 (segment (start 46.0555 12.9919) (end 43.8463 15.2011) (width 0.2) (layer "B.Cu") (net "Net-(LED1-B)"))
 (segment (start 40.9483 20.1391) (end 41.1342 20.325) (width 0.2) (layer "B.Cu") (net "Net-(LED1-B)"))
 (segment (start 40.9483 17.2124) (end 40.9483 20.1391) (width 0.2) (layer "B.Cu") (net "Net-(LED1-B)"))
 (segment (start 50.1679 14.59) (end 50.4685 14.2894) (width 0.2) (layer "B.Cu") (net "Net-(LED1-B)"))
 (segment (start 48.7584 12.9919) (end 46.0555 12.9919) (width 0.2) (layer "B.Cu") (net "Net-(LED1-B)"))
 (segment (start 49.6698 13.4081) (end 49.1746 13.4081) (width 0.2) (layer "B.Cu") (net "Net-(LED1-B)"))
 (segment (start 45.0875 13.3527) (end 46.6172 14.8824) (width 0.2) (layer "F.Cu") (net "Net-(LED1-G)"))
 (segment (start 47.25 17.55) (end 47.25 18.0411) (width 0.2) (layer "F.Cu") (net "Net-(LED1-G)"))
 (segment (start 43.6854 17.9736) (end 43.6854 18.3285) (width 0.2) (layer "F.Cu") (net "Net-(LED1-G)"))
 (segment (start 45.0875 13) (end 45.0875 13.3527) (width 0.2) (layer "F.Cu") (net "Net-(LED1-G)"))
 (segment (start 43.6854 18.3285) (end 46.1089 20.752) (width 0.2) (layer "F.Cu") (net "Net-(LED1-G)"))
 (segment (start 47.25 18.0411) (end 46.8248 18.4663) (width 0.2) (layer "F.Cu") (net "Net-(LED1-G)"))
 (via (at 43.6854 17.9736) (size 0.6) (drill 0.3) (layers "F.Cu" "B.Cu") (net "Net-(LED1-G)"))
 (via (at 46.6172 14.8824) (size 0.6) (drill 0.3) (layers "F.Cu" "B.Cu") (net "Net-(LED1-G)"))
 (via (at 46.1089 20.752) (size 0.6) (drill 0.3) (layers "F.Cu" "B.Cu") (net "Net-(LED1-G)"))
 (via (at 46.8248 18.4663) (size 0.6) (drill 0.3) (layers "F.Cu" "B.Cu") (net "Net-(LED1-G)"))
 (segment (start 46.8248 18.4663) (end 46.1089 19.1822) (width 0.2) (layer "B.Cu") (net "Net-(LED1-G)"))
 (segment (start 44.2899 17.3691) (end 43.6854 17.9736) (width 0.2) (layer "B.Cu") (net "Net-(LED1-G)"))
 (segment (start 47.7323 16.3316) (end 46.6948 17.3691) (width 0.2) (layer "B.Cu") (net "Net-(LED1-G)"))
 (segment (start 47.0623 14.8824) (end 47.7323 15.5524) (width 0.2) (layer "B.Cu") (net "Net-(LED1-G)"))
 (segment (start 46.1089 19.1822) (end 46.1089 20.752) (width 0.2) (layer "B.Cu") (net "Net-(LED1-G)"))
 (segment (start 46.6948 17.3691) (end 44.2899 17.3691) (width 0.2) (layer "B.Cu") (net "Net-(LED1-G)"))
 (segment (start 46.6172 14.8824) (end 47.0623 14.8824) (width 0.2) (layer "B.Cu") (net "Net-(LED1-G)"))
 (segment (start 47.7323 15.5524) (end 47.7323 16.3316) (width 0.2) (layer "B.Cu") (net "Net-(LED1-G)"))
 (segment (start 47.25 16.45) (end 47.25 14.3375) (width 0.2) (layer "F.Cu") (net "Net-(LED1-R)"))
 (segment (start 47.25 14.3375) (end 48.5875 13) (width 0.2) (layer "F.Cu") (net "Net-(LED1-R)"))
 (segment (start 47.6042 20.4324) (end 46.6643 20.4324) (width 0.2) (layer "F.Cu") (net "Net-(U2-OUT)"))
 (segment (start 48.55 22.5914) (end 48.55 21.3782) (width 0.2) (layer "F.Cu") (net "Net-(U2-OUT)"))
 (segment (start 49.3889 23.4303) (end 48.55 22.5914) (width 0.2) (layer "F.Cu") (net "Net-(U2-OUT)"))
 (segment (start 46.6643 20.4324) (end 44.4924 18.2605) (width 0.2) (layer "F.Cu") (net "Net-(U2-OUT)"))
 (segment (start 48.55 21.3782) (end 47.6042 20.4324) (width 0.2) (layer "F.Cu") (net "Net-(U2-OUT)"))
 (segment (start 53 22) (end 53 22.284) (width 0.2) (layer "F.Cu") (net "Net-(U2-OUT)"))
 (segment (start 44.4924 18.2605) (end 44.4924 16.0037) (width 0.2) (layer "F.Cu") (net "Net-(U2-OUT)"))
 (segment (start 44.4924 16.0037) (end 45.0116 15.4845) (width 0.2) (layer "F.Cu") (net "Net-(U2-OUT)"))
 (segment (start 53 22.284) (end 51.8537 23.4303) (width 0.2) (layer "F.Cu") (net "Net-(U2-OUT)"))
 (segment (start 51.8537 23.4303) (end 49.3889 23.4303) (width 0.2) (layer "F.Cu") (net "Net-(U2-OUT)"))
 (via (at 45.0116 15.4845) (size 0.6) (drill 0.3) (layers "F.Cu" "B.Cu") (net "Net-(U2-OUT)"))
 (segment (start 46.4461 14.05) (end 45.0116 15.4845) (width 0.2) (layer "B.Cu") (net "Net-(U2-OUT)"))
 (segment (start 46.9 14.05) (end 46.4461 14.05) (width 0.2) (layer "B.Cu") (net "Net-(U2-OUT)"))
 (segment (start 48.8549 14.05) (end 49.1 14.05) (width 0.2) (layer "B.Cu") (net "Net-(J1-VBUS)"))
 (segment (start 48.4711 14.4338) (end 48.8549 14.05) (width 0.2) (layer "B.Cu") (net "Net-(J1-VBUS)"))
 (segment (start 46.2513 13.3936) (end 47.4309 13.3936) (width 0.2) (layer "B.Cu") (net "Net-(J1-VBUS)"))
 (segment (start 60.2383 17.42) (end 58.7683 15.95) (width 0.2) (layer "B.Cu") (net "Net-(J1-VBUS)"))
 (segment (start 58.7683 15.95) (end 49.1 15.95) (width 0.2) (layer "B.Cu") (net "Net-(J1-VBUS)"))
 (segment (start 44.35 16.5) (end 44.35 15.2949) (width 0.2) (layer "B.Cu") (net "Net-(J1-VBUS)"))
 (segment (start 47.4309 13.3936) (end 48.4711 14.4338) (width 0.2) (layer "B.Cu") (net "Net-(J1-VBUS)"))
 (segment (start 49.1 15.95) (end 48.7863 15.95) (width 0.2) (layer "B.Cu") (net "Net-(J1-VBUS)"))
 (segment (start 44.35 15.2949) (end 46.2513 13.3936) (width 0.2) (layer "B.Cu") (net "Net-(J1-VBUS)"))
 (segment (start 48.7863 15.95) (end 48.2288 15.3925) (width 0.2) (layer "B.Cu") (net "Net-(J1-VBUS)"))
 (segment (start 48.2288 15.3925) (end 48.2288 14.6761) (width 0.2) (layer "B.Cu") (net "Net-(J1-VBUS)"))
 (segment (start 48.2288 14.6761) (end 48.4711 14.4338) (width 0.2) (layer "B.Cu") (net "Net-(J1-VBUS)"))
 (segment (start 62.04 17.42) (end 60.2383 17.42) (width 0.2) (layer "B.Cu") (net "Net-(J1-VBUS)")))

